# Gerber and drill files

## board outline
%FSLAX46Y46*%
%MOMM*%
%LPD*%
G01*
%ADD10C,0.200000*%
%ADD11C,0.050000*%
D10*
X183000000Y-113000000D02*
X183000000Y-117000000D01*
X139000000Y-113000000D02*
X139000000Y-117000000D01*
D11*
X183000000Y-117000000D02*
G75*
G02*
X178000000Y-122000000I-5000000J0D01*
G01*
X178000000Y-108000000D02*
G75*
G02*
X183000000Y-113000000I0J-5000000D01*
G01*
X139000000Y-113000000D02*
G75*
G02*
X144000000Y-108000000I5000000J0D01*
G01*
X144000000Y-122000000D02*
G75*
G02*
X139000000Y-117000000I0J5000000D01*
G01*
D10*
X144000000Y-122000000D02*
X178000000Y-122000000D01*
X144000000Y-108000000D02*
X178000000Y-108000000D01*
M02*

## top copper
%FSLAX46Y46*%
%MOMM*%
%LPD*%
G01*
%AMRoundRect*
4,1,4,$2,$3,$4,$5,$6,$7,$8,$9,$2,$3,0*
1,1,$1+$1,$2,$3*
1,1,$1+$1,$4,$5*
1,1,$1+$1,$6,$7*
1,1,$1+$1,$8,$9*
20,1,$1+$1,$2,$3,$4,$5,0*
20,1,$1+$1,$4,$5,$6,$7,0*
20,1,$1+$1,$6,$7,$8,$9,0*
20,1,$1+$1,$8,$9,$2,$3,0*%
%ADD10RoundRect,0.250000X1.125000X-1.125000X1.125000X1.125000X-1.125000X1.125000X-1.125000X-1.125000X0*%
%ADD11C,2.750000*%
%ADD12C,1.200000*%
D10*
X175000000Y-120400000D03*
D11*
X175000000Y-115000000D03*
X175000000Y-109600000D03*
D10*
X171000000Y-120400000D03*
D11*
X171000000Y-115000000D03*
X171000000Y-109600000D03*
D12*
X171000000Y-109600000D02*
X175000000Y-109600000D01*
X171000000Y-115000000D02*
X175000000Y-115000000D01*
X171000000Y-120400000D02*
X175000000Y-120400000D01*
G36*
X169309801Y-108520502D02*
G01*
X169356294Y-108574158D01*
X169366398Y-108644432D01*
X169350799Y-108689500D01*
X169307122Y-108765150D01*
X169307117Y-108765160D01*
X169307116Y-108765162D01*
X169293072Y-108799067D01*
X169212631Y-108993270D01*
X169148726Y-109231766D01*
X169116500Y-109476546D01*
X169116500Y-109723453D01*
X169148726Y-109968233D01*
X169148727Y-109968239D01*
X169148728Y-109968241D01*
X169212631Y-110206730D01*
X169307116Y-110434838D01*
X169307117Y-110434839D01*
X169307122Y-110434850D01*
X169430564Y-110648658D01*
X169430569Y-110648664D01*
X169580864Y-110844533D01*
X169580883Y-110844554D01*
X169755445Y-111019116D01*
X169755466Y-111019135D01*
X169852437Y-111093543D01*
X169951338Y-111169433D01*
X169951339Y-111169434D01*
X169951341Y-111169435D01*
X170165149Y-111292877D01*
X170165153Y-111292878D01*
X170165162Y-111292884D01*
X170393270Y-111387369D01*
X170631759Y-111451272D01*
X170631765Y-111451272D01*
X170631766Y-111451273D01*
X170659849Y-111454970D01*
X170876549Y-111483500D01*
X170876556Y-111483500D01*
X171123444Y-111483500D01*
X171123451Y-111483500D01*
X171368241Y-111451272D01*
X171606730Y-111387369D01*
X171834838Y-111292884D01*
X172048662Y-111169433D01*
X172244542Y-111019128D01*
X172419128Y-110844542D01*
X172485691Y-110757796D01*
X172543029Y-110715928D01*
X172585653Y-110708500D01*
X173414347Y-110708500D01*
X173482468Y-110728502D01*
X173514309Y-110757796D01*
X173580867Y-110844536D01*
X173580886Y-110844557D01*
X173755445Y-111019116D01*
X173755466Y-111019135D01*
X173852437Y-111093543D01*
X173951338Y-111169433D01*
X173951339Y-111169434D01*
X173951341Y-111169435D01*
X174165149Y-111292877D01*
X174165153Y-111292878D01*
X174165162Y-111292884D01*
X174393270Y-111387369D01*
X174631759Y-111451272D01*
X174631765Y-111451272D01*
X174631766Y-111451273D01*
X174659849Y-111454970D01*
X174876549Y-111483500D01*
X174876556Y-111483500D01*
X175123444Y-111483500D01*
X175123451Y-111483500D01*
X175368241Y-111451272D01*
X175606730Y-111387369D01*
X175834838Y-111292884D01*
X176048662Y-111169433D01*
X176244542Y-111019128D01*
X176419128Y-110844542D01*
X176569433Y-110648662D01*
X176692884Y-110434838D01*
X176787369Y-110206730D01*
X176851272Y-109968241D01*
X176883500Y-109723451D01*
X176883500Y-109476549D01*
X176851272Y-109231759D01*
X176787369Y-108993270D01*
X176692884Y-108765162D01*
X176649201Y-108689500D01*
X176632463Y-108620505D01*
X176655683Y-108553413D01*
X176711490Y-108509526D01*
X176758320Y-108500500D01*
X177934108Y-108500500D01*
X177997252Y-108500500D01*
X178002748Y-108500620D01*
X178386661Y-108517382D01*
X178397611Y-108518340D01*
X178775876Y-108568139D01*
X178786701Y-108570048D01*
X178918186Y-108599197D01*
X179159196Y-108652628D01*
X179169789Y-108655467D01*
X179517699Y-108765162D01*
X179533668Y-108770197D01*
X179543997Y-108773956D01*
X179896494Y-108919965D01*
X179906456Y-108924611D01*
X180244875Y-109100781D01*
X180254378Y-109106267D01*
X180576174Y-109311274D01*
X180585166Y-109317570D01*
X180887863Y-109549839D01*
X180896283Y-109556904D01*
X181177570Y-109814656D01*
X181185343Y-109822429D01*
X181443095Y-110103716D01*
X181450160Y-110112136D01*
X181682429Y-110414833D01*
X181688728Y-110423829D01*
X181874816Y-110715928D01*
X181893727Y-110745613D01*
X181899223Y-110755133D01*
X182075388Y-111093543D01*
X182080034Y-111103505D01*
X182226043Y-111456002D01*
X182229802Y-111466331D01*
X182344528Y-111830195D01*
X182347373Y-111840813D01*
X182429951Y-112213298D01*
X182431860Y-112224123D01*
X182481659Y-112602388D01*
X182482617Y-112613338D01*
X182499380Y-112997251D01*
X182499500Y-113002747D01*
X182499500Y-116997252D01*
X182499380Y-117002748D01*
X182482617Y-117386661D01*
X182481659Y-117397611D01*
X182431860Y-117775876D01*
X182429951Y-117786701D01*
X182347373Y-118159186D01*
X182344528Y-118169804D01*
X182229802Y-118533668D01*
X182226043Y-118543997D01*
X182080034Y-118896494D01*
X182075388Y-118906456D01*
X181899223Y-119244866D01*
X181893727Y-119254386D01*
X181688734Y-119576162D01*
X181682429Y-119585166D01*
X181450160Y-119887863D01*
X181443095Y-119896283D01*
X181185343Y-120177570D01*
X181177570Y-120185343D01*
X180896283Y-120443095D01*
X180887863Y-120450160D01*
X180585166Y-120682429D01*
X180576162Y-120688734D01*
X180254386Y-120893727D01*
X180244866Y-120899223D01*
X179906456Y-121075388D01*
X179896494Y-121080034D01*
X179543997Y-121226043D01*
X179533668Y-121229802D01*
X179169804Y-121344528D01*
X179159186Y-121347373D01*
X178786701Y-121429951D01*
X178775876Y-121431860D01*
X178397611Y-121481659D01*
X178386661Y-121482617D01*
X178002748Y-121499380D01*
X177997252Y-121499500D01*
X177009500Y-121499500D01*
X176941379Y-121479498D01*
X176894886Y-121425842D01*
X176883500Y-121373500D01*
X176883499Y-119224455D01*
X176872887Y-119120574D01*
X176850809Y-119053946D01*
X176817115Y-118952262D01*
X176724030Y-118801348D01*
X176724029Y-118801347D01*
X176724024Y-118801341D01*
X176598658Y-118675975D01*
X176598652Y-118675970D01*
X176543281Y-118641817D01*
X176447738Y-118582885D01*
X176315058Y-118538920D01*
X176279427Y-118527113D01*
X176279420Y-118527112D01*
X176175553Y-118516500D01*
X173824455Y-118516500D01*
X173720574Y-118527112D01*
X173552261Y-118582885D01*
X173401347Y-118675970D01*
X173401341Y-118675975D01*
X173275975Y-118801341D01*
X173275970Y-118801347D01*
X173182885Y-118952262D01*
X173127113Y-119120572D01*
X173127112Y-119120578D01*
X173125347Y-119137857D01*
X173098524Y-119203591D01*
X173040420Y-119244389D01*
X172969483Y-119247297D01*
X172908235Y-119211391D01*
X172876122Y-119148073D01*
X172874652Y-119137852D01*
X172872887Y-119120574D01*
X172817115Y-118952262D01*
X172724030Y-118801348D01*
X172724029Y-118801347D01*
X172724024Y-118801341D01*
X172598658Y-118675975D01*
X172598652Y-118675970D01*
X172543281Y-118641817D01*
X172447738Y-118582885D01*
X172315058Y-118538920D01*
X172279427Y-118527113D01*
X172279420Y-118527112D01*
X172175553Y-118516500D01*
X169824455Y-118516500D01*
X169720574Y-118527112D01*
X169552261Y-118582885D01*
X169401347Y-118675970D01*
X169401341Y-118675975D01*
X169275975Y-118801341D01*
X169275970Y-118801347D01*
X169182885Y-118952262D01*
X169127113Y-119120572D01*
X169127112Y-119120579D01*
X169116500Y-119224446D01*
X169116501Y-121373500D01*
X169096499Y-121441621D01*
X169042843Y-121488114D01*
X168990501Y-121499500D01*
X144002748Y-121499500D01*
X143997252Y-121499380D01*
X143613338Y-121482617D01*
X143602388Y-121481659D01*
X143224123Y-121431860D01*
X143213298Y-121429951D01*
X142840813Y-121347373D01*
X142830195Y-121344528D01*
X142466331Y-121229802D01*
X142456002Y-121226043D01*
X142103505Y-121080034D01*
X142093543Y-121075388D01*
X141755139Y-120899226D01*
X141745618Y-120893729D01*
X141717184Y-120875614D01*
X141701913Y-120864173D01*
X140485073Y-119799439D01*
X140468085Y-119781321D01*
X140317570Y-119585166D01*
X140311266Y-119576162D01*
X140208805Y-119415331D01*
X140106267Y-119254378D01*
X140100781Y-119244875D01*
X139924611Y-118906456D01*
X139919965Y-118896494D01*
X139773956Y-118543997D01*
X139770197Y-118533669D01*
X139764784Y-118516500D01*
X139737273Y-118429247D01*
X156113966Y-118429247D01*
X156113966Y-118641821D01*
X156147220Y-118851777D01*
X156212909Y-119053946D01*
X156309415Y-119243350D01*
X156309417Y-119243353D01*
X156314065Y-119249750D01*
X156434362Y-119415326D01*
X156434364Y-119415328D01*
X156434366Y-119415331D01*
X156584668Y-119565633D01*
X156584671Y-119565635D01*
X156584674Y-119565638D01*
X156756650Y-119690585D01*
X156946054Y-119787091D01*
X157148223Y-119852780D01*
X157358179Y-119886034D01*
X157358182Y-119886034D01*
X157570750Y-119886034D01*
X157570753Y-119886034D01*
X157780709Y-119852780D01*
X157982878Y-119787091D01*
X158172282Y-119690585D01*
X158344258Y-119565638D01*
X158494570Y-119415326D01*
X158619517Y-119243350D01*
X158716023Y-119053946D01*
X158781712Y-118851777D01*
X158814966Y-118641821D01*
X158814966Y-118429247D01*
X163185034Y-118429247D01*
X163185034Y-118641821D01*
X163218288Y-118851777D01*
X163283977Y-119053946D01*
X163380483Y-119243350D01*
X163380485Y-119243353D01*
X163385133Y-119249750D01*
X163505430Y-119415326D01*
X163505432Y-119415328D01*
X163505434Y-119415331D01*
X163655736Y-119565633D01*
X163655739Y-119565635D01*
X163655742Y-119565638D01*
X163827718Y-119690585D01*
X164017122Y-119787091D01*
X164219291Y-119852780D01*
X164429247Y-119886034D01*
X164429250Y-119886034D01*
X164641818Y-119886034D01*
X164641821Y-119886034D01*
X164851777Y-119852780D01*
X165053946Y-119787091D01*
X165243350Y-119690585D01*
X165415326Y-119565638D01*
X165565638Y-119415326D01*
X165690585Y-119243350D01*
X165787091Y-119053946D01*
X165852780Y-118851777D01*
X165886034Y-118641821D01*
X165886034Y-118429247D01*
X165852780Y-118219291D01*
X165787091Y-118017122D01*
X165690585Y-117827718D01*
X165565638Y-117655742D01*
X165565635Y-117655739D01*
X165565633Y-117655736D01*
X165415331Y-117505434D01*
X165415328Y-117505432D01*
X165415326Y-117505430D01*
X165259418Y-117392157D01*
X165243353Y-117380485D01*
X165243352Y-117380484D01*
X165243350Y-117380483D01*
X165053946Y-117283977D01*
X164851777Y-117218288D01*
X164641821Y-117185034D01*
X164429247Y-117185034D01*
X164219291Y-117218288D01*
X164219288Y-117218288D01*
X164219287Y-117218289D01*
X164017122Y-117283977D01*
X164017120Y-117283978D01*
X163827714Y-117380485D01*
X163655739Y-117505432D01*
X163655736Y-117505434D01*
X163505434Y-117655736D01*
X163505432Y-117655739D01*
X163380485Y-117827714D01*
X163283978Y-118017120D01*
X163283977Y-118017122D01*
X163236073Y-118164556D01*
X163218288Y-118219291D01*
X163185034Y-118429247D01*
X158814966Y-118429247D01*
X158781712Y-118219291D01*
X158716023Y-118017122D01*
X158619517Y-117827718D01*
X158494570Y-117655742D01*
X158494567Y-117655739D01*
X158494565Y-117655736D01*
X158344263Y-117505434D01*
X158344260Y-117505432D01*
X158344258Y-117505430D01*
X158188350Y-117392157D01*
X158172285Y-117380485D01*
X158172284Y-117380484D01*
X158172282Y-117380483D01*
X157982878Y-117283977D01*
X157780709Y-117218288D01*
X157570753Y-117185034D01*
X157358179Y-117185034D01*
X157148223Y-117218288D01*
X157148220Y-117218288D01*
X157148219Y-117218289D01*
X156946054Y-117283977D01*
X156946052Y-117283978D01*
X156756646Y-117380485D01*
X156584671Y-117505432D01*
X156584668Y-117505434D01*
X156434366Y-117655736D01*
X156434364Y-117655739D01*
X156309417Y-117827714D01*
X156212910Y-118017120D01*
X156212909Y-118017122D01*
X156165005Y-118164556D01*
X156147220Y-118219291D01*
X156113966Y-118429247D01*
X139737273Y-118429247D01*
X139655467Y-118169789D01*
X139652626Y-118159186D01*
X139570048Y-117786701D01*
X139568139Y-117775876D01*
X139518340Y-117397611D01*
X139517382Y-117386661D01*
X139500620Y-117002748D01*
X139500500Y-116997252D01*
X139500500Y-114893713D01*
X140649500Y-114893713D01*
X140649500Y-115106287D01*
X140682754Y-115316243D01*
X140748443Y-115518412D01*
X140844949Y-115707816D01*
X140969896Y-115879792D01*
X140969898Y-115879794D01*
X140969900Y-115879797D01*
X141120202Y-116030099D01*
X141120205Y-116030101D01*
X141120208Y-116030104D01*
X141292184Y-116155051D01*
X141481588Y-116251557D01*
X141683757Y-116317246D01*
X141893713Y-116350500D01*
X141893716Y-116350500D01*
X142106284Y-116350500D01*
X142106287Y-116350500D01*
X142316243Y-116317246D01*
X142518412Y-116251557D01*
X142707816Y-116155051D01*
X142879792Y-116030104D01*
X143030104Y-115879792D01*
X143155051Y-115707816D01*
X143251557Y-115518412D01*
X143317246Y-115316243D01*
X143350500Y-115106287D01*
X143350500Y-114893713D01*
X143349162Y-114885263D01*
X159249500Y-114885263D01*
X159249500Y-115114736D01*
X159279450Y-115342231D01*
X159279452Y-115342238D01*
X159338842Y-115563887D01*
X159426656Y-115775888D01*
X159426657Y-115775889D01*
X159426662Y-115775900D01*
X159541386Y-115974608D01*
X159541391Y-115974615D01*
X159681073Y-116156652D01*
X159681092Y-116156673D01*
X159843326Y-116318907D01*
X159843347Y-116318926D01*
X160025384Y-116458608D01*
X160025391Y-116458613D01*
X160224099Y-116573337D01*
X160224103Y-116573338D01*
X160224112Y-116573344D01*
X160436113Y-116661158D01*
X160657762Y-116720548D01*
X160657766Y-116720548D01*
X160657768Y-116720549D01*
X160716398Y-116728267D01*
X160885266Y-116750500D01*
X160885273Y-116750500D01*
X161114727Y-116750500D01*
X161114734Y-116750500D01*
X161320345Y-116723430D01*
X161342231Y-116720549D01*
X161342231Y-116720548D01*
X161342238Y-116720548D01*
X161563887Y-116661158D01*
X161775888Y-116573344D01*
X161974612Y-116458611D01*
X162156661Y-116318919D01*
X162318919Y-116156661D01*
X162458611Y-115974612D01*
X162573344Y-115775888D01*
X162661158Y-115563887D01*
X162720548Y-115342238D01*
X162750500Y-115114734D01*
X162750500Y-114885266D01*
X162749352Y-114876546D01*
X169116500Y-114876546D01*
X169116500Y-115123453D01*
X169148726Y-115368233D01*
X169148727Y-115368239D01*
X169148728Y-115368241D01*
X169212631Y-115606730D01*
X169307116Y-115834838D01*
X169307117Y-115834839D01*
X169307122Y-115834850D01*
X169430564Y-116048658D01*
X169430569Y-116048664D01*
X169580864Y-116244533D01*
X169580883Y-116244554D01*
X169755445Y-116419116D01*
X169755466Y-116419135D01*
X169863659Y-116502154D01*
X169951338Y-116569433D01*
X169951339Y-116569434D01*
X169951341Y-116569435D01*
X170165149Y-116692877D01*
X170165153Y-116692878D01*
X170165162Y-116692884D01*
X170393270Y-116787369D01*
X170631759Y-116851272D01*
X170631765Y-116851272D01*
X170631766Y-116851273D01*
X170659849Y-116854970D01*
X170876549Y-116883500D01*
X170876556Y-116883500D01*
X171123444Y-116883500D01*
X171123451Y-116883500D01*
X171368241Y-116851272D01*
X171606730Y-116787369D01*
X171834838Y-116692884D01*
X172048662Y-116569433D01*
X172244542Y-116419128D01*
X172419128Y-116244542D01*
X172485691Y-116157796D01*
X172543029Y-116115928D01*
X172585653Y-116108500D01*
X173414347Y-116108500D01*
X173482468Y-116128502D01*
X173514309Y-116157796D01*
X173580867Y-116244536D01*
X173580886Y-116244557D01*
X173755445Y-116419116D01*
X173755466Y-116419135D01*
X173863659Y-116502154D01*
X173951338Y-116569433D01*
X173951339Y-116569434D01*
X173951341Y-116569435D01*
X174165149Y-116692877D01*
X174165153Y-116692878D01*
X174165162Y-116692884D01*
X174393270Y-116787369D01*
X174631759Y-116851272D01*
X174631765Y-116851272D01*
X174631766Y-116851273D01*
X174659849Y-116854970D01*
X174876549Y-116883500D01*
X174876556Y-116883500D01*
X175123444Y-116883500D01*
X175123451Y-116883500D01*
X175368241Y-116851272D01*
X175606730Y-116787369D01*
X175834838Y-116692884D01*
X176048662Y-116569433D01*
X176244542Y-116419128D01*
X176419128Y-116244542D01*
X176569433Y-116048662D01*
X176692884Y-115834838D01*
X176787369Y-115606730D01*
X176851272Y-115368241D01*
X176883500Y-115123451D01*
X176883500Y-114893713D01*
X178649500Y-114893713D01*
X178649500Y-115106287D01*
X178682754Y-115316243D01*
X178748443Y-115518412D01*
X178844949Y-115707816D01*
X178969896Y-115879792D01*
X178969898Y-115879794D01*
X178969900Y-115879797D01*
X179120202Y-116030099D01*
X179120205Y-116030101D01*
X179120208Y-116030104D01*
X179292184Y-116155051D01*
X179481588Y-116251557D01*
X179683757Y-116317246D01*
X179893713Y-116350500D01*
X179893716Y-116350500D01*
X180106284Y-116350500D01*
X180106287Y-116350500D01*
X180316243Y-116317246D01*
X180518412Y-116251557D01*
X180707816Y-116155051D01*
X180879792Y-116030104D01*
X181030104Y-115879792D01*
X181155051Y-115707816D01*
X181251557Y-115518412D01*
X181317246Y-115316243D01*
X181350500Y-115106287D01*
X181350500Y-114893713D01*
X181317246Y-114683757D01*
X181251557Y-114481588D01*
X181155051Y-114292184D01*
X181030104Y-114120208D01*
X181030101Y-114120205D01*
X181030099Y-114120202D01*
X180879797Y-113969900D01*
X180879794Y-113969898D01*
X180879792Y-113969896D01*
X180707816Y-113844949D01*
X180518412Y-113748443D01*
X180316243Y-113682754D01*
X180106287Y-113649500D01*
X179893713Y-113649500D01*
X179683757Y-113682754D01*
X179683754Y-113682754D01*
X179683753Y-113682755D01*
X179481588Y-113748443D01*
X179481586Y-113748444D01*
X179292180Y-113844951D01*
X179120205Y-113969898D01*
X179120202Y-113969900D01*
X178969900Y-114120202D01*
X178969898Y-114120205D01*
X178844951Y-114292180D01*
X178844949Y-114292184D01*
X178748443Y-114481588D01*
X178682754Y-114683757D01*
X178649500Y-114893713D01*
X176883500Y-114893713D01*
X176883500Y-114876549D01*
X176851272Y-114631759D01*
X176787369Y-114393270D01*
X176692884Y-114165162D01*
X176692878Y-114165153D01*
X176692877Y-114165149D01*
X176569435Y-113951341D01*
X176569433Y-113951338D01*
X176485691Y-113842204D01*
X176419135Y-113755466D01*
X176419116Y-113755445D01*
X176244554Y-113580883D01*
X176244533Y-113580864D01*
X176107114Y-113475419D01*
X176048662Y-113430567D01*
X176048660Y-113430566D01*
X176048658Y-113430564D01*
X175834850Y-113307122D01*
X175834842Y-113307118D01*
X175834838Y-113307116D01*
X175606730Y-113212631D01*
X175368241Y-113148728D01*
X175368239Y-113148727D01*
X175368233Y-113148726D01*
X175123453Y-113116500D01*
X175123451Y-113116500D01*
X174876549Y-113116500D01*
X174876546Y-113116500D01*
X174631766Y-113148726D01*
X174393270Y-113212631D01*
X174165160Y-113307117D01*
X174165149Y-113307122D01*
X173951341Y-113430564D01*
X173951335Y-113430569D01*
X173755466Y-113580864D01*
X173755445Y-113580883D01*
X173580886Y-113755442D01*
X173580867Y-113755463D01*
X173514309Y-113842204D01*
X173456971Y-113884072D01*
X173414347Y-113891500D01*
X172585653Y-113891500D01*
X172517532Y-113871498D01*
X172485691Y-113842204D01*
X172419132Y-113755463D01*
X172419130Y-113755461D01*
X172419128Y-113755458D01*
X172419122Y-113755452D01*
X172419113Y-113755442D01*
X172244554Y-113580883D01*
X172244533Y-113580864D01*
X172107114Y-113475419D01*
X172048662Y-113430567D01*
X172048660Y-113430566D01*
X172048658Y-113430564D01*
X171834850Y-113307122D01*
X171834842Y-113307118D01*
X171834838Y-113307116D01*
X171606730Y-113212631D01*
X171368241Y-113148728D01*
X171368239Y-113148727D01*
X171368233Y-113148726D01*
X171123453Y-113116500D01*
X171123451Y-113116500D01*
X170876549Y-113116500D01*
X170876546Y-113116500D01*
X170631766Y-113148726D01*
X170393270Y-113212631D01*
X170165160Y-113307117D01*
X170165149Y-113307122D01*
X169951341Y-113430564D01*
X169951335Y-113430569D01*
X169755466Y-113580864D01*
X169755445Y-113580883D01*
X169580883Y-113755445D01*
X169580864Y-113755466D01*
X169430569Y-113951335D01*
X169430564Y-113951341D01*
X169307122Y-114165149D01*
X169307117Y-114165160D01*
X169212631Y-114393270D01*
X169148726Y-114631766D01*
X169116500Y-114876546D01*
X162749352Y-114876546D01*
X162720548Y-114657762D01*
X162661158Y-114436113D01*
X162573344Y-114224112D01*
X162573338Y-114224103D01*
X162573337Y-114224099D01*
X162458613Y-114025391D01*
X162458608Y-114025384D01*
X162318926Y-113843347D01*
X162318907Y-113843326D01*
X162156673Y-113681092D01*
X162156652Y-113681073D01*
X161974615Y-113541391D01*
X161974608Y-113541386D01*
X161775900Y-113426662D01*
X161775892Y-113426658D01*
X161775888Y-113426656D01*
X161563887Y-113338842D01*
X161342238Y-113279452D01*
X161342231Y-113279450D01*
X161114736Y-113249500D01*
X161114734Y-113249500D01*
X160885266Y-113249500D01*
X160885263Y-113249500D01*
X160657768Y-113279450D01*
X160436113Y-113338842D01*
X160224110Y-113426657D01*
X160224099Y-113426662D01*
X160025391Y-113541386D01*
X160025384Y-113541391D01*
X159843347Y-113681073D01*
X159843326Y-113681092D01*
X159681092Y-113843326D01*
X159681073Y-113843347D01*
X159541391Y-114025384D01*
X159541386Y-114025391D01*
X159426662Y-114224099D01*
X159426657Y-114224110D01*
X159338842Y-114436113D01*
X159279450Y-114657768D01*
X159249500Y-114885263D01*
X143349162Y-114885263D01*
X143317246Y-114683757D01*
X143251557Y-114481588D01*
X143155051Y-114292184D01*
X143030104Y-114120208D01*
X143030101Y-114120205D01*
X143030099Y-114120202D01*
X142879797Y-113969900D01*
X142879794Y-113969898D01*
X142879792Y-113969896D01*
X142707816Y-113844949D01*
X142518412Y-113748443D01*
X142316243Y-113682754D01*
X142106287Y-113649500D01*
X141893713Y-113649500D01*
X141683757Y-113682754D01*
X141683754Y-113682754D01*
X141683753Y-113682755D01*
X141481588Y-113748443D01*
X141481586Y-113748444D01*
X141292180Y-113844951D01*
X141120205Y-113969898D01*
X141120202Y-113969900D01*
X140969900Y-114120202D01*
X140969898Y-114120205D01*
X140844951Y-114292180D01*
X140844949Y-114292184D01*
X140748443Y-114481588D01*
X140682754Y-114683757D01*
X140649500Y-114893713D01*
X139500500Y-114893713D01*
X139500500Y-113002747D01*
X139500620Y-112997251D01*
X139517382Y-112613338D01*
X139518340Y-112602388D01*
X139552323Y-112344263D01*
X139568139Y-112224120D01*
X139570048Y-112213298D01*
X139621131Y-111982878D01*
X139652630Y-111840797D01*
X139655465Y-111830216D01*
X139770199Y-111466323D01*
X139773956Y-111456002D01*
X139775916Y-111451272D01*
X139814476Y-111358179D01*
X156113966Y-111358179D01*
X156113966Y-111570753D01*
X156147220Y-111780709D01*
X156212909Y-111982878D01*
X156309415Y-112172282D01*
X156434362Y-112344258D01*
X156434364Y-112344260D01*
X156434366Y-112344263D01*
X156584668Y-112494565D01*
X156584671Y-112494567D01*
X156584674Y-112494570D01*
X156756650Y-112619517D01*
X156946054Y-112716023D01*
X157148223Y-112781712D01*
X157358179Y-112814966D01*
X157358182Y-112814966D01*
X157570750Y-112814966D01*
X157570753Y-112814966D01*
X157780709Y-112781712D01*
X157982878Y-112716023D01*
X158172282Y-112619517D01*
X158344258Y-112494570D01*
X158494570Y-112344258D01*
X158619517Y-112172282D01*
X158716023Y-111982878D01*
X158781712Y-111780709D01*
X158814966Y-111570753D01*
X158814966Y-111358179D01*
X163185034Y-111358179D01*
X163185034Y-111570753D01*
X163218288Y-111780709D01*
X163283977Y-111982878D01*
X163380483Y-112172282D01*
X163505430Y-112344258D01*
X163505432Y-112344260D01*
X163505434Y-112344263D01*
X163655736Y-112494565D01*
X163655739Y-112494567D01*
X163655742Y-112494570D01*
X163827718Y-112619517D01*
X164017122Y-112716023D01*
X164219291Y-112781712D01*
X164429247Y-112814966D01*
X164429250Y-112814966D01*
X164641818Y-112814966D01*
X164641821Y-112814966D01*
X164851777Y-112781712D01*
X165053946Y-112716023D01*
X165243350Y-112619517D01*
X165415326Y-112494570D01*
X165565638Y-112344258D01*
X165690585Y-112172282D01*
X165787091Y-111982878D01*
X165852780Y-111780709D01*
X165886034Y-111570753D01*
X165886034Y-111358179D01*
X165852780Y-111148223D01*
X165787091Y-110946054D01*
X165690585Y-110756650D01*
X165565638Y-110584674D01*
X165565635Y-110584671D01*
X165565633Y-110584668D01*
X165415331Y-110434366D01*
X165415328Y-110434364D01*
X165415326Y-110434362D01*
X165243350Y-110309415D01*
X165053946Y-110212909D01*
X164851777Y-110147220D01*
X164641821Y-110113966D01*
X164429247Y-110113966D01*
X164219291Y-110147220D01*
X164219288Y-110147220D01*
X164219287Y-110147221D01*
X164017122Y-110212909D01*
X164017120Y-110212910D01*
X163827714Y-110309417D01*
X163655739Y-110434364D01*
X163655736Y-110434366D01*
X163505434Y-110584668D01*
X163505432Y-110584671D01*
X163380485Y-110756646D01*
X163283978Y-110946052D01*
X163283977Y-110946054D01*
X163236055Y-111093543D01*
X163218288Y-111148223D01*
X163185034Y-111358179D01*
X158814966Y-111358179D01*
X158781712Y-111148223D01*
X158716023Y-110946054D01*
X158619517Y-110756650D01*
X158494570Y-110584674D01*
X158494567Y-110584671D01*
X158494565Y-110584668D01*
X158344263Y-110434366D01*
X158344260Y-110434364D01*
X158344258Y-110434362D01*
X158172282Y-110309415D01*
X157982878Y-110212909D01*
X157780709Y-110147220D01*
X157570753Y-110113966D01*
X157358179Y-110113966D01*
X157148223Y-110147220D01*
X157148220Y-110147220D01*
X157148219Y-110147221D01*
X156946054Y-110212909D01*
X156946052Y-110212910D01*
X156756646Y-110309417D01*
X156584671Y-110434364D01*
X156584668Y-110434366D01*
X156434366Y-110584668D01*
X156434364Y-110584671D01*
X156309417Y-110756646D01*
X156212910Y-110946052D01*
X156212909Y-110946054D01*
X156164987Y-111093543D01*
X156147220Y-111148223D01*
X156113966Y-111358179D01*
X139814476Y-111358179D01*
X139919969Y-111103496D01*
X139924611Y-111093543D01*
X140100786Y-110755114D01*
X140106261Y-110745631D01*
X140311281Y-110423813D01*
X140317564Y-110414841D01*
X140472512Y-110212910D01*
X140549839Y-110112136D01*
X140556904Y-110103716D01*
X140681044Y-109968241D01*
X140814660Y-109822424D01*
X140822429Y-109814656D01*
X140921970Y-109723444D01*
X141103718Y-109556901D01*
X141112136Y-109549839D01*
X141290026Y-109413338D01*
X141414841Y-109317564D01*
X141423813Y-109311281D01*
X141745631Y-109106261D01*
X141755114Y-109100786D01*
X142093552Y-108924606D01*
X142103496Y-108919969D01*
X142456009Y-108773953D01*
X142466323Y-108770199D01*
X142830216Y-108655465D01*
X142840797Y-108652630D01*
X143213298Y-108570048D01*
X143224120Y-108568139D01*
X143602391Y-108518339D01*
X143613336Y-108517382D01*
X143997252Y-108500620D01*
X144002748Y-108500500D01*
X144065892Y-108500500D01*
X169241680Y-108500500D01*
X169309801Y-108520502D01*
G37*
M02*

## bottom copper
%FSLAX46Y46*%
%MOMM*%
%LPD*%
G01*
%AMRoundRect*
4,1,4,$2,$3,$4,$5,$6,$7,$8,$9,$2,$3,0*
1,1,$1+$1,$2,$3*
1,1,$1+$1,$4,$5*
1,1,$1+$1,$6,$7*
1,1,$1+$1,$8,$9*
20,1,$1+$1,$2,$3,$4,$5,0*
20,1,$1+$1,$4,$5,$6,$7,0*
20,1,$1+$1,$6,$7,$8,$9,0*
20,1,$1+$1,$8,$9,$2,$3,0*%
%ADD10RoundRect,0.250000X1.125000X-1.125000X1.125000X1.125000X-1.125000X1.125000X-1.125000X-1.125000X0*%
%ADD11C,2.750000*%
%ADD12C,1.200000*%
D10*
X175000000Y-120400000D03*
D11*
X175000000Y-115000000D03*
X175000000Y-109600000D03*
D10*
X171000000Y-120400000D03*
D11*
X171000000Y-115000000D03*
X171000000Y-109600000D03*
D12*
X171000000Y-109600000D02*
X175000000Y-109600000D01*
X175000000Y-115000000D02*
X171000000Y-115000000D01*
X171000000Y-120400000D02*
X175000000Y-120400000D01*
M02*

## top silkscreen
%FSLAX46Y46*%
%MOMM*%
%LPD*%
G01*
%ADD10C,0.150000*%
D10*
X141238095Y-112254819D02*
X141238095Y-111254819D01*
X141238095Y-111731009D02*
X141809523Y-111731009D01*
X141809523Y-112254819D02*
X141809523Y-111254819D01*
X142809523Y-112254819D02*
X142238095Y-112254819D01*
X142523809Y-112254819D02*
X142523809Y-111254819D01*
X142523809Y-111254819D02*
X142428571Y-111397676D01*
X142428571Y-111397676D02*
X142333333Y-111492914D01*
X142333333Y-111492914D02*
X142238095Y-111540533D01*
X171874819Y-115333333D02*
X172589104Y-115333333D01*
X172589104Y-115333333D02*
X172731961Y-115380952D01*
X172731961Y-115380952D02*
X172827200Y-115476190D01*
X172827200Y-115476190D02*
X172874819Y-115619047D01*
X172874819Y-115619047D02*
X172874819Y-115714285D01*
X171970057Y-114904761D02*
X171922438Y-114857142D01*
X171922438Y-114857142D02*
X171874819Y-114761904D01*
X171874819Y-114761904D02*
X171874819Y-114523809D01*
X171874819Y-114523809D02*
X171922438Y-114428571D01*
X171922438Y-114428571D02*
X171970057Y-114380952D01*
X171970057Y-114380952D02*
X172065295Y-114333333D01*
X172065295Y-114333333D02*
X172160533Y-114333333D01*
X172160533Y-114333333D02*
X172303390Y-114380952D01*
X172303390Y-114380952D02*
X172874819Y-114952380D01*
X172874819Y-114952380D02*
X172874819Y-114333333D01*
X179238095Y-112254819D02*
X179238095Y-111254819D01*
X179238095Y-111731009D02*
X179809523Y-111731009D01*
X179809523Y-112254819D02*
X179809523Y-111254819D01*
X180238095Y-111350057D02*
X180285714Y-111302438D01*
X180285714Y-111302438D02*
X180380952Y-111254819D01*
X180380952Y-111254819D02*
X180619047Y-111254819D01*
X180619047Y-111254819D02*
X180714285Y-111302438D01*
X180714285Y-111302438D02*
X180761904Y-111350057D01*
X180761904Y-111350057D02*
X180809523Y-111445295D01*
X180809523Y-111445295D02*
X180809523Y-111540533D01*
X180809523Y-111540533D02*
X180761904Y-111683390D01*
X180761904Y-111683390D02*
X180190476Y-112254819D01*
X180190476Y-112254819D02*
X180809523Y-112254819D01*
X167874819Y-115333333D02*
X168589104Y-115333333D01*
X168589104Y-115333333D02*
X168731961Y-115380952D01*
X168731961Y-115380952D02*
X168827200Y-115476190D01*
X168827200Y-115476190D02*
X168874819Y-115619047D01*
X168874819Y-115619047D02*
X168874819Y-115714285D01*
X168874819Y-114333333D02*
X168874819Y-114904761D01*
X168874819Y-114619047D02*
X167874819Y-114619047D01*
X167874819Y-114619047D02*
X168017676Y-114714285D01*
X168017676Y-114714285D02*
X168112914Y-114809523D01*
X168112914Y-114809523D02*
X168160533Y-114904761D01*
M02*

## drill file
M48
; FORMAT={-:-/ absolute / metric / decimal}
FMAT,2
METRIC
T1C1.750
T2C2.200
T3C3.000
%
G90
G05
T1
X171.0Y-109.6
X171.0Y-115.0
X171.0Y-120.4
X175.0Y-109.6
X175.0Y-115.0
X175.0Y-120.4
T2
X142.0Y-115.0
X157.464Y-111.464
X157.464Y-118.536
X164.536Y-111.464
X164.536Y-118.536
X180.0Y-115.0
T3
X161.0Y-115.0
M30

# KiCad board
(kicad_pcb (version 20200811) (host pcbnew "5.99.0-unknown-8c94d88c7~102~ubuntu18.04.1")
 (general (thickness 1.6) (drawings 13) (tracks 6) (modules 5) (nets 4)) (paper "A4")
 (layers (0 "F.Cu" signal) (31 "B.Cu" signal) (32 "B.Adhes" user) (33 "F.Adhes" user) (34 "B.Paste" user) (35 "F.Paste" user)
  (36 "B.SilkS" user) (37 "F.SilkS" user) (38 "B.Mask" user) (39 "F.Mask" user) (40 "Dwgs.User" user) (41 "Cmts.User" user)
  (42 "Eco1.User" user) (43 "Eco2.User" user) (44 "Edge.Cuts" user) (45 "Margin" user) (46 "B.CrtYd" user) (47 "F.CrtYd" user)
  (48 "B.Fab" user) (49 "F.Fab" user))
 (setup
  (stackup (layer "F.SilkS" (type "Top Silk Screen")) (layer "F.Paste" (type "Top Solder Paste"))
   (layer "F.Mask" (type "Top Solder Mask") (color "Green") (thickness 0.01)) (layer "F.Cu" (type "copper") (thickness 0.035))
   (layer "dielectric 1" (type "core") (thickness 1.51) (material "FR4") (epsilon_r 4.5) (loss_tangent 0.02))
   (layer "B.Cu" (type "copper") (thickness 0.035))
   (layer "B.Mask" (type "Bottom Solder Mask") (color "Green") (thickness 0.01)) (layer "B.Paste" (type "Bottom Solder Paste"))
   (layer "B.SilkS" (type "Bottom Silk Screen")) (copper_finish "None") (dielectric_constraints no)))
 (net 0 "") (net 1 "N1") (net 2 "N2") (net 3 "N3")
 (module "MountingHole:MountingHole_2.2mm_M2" (layer "F.Cu") (at 142 115)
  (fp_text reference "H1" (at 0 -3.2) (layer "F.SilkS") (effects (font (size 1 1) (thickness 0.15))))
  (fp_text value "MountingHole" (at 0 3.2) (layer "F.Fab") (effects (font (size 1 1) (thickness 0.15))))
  (pad "1" np_thru_hole circle (at 0 0) (size 2.2 2.2) (drill 2.2) (layers *.Cu *.Mask)))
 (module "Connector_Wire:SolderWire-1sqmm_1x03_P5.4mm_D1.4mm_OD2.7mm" (layer "F.Cu") (at 175 120.4 90)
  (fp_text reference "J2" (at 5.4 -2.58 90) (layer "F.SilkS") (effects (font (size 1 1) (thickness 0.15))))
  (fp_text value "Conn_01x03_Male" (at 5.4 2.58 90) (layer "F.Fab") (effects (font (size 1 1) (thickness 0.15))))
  (pad "1" thru_hole roundrect (at 0 0 90) (size 2.75 2.75) (drill 1.75) (layers *.Cu *.Mask) (remove_unused_layers) (keep_end_layers)
   (roundrect_rratio 0.090909) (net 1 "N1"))
  (pad "2" thru_hole circle (at 5.4 0 90) (size 2.75 2.75) (drill 1.75) (layers *.Cu *.Mask) (remove_unused_layers) (keep_end_layers)
   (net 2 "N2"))
  (pad "3" thru_hole circle (at 10.8 0 90) (size 2.75 2.75) (drill 1.75) (layers *.Cu *.Mask) (remove_unused_layers) (keep_end_layers)
   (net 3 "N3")))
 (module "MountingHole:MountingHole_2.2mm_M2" (layer "F.Cu") (at 180 115)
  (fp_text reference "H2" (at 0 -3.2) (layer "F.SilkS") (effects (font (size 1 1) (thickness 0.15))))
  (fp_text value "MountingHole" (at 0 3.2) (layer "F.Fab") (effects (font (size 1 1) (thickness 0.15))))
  (pad "1" np_thru_hole circle (at 0 0) (size 2.2 2.2) (drill 2.2) (layers *.Cu *.Mask)))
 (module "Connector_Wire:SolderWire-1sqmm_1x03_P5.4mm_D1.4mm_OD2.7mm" (layer "F.Cu") (at 171 120.4 90)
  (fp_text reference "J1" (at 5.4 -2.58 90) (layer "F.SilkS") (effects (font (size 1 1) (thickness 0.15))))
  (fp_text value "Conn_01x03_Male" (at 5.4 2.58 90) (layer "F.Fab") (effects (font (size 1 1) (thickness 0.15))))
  (pad "1" thru_hole roundrect (at 0 0 90) (size 2.75 2.75) (drill 1.75) (layers *.Cu *.Mask) (roundrect_rratio 0.090909) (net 1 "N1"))
  (pad "2" thru_hole circle (at 5.4 0 90) (size 2.75 2.75) (drill 1.75) (layers *.Cu *.Mask) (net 2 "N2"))
  (pad "3" thru_hole circle (at 10.8 0 90) (size 2.75 2.75) (drill 1.75) (layers *.Cu *.Mask) (remove_unused_layers) (keep_end_layers)
   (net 3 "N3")))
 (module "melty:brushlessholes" (layer "F.Cu") (at 161 115 45)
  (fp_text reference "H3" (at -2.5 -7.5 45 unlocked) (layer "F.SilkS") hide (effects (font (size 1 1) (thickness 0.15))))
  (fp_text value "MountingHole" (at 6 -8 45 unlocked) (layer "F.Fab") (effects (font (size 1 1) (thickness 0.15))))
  (pad "" np_thru_hole circle (at 0 5 45) (size 2.2 2.2) (drill 2.2) (layers *.Cu *.Mask))
  (pad "" np_thru_hole circle (at 0 0 45) (size 3 3) (drill 3) (layers *.Cu *.Mask))
  (pad "" np_thru_hole circle (at 5 0 45) (size 2.2 2.2) (drill 2.2) (layers *.Cu *.Mask))
  (pad "" np_thru_hole circle (at 0 -5 45) (size 2.2 2.2) (drill 2.2) (layers *.Cu *.Mask))
  (pad "" np_thru_hole circle (at -5 0 45) (size 2.2 2.2) (drill 2.2) (layers *.Cu *.Mask)))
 (gr_line (start 183 113) (end 183 117) (layer "Edge.Cuts") (width 0.2))
 (gr_line (start 139 113) (end 139 117) (layer "Edge.Cuts") (width 0.2))
 (gr_arc (start 178 117) (end 183 117) (angle 90) (layer "Edge.Cuts") (width 0.05))
 (gr_arc (start 178 113) (end 178 108) (angle 90) (layer "Edge.Cuts") (width 0.05))
 (gr_arc (start 144 113) (end 139 113) (angle 90) (layer "Edge.Cuts") (width 0.05))
 (gr_arc (start 144 117) (end 144 122) (angle 90) (layer "Edge.Cuts") (width 0.05))
 (gr_line (start 144 122) (end 178 122) (layer "Edge.Cuts") (width 0.2))
 (gr_line (start 144 108) (end 178 108) (layer "Edge.Cuts") (width 0.2))
 (segment (start 171 109.6) (end 175 109.6) (width 1.2) (layer "F.Cu") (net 3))
 (segment (start 171 109.6) (end 175 109.6) (width 1.2) (layer "B.Cu") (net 3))
 (segment (start 171 115) (end 175 115) (width 1.2) (layer "F.Cu") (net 2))
 (segment (start 175 115) (end 171 115) (width 1.2) (layer "B.Cu") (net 2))
 (segment (start 171 120.4) (end 175 120.4) (width 1.2) (layer "F.Cu") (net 1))
 (segment (start 171 120.4) (end 175 120.4) (width 1.2) (layer "B.Cu") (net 1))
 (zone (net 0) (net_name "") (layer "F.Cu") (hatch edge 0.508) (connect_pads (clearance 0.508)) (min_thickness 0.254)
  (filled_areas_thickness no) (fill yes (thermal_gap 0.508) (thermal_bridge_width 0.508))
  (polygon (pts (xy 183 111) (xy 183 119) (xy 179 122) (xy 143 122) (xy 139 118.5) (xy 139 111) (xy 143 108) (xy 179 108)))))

